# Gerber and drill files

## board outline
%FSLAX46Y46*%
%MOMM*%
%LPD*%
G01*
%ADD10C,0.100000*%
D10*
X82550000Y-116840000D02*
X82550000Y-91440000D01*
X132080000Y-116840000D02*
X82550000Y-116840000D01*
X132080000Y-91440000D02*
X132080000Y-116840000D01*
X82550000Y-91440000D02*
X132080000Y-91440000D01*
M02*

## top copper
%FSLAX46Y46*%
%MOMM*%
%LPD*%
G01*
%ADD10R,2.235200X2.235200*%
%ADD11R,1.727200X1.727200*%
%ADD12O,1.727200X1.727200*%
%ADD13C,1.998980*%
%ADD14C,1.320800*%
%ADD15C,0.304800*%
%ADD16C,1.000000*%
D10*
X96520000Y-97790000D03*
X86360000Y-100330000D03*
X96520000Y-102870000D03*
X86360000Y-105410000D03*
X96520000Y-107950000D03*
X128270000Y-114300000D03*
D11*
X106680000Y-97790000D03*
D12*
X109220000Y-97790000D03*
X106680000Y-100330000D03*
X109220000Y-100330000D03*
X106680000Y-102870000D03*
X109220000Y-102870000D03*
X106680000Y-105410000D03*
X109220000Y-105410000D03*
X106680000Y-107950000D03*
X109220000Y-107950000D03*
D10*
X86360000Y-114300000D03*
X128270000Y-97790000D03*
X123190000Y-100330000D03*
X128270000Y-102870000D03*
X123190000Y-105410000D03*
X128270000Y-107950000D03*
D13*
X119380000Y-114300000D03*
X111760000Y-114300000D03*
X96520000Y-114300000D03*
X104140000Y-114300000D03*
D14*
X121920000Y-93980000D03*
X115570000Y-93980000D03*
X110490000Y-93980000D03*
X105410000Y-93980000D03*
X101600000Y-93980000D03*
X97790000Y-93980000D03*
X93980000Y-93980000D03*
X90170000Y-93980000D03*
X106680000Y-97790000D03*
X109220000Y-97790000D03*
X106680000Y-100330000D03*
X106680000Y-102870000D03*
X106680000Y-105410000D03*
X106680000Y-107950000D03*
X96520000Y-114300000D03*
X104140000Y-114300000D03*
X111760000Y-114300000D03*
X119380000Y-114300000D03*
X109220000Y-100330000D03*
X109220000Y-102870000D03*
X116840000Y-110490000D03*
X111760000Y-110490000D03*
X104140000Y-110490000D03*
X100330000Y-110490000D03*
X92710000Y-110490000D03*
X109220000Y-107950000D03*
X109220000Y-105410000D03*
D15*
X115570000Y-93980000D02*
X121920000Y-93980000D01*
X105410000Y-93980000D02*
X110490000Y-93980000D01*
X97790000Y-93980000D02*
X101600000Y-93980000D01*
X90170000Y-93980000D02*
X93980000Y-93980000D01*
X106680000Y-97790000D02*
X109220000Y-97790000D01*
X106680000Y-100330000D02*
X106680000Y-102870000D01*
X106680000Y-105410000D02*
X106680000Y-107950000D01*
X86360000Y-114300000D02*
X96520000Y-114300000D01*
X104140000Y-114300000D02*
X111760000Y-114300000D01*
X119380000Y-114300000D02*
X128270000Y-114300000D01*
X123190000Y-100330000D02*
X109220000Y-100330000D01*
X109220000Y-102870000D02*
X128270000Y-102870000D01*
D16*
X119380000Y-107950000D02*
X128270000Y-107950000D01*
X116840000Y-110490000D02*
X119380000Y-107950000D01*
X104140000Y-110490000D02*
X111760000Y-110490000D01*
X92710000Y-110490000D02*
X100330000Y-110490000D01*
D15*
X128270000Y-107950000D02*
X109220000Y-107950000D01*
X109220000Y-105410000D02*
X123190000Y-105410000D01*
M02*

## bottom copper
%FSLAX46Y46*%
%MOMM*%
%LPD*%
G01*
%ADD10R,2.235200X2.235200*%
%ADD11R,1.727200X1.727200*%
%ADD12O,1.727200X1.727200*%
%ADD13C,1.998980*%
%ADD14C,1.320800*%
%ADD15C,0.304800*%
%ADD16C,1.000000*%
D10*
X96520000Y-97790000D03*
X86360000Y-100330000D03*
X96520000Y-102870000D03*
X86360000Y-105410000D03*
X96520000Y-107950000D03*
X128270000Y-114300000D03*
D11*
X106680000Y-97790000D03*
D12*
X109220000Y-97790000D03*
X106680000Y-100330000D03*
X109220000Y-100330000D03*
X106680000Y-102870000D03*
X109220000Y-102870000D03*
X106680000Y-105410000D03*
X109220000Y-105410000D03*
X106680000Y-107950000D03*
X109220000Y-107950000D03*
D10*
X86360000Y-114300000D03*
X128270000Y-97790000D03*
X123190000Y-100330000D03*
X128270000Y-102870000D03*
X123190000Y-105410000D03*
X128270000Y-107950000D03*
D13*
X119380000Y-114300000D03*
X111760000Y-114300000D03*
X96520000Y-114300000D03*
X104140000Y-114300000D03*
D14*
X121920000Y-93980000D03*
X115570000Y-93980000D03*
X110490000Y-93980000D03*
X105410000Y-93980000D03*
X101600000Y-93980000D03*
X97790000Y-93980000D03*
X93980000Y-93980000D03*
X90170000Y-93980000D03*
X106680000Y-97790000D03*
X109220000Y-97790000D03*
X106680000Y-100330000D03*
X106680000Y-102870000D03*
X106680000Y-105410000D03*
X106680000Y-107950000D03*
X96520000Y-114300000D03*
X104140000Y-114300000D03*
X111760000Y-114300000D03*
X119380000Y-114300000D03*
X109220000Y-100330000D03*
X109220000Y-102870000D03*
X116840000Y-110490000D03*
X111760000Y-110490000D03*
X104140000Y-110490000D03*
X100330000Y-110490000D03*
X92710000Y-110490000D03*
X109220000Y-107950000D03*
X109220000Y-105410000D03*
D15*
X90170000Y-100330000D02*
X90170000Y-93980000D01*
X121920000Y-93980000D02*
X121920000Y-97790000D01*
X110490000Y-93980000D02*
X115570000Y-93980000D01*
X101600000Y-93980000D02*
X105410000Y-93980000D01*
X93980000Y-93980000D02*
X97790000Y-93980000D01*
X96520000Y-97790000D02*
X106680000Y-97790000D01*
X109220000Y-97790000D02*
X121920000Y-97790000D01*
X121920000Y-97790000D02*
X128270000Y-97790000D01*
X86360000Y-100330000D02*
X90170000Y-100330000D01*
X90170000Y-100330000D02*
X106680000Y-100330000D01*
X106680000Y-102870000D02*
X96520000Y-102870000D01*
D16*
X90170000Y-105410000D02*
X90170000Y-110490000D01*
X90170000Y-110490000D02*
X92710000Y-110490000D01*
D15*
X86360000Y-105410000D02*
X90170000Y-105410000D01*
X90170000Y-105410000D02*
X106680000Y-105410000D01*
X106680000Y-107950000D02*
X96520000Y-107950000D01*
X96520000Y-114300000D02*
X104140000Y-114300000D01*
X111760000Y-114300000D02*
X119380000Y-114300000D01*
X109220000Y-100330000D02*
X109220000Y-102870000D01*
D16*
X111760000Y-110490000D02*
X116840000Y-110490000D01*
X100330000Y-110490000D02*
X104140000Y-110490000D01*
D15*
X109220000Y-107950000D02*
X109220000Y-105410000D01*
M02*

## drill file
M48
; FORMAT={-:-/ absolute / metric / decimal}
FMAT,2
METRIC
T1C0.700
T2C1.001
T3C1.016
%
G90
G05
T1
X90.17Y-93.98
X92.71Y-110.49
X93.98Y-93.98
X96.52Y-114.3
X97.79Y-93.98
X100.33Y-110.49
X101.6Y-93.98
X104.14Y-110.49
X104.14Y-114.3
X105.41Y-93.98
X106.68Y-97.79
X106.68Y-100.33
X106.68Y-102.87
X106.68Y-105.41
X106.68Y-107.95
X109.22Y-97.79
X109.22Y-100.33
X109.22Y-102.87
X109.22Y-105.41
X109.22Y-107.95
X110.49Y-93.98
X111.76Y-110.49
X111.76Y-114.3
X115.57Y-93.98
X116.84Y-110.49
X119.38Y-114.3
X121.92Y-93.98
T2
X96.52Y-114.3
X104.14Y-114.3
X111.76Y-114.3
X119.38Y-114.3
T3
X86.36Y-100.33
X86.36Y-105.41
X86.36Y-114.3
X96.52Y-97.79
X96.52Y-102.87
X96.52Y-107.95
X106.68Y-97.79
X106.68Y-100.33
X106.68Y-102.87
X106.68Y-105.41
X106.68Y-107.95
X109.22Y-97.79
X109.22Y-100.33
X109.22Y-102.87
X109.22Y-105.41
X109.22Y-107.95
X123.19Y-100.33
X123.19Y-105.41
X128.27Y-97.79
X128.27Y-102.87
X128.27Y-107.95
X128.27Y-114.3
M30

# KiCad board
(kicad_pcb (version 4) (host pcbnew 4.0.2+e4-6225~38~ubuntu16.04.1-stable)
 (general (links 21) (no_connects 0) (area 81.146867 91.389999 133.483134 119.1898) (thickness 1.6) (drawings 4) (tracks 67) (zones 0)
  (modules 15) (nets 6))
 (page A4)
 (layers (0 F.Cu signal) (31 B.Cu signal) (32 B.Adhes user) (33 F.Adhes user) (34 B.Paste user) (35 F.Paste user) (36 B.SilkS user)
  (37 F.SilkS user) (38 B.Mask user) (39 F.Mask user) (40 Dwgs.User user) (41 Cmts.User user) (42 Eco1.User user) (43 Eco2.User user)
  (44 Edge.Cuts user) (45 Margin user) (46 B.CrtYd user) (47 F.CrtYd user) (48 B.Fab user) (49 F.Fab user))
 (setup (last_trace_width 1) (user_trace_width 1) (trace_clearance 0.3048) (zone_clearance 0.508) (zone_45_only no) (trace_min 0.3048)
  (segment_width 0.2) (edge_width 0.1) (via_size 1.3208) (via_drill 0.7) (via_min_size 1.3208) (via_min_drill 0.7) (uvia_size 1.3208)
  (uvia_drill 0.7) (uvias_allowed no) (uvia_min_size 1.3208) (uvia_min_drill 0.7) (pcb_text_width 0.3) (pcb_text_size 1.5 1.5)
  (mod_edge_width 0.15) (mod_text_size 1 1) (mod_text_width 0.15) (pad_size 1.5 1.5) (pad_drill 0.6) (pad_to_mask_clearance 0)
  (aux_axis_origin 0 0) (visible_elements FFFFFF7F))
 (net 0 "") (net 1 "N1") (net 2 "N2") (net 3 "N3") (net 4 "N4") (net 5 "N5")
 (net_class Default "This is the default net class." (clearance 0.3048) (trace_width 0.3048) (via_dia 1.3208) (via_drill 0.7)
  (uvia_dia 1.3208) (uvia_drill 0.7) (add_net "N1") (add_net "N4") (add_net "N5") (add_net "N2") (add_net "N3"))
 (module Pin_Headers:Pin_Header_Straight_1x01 (layer F.Cu) (at 96.52 97.79)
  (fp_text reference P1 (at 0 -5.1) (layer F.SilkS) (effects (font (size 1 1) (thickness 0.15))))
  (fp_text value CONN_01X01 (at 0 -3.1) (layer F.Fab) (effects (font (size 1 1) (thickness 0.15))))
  (pad 1 thru_hole rect (at 0 0) (size 2.2352 2.2352) (drill 1.016) (layers *.Cu *.Mask F.SilkS) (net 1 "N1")))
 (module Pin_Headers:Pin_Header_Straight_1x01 (layer F.Cu) (at 86.36 100.33)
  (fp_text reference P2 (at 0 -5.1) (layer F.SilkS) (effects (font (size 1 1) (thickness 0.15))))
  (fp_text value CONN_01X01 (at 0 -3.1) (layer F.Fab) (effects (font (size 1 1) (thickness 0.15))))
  (pad 1 thru_hole rect (at 0 0) (size 2.2352 2.2352) (drill 1.016) (layers *.Cu *.Mask F.SilkS) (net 1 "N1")))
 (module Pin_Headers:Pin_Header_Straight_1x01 (layer F.Cu) (at 96.52 102.87)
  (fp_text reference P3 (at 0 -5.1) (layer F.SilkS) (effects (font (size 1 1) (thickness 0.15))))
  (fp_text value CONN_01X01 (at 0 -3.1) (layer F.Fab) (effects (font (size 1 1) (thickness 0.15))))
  (pad 1 thru_hole rect (at 0 0) (size 2.2352 2.2352) (drill 1.016) (layers *.Cu *.Mask F.SilkS) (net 1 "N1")))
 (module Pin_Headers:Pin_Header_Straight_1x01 (layer F.Cu) (at 86.36 105.41)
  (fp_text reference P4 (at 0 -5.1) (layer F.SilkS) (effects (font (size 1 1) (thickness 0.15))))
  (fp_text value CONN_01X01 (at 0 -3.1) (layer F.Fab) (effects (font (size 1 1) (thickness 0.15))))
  (pad 1 thru_hole rect (at 0 0) (size 2.2352 2.2352) (drill 1.016) (layers *.Cu *.Mask F.SilkS) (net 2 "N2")))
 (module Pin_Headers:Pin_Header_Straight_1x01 (layer F.Cu) (at 96.52 107.95)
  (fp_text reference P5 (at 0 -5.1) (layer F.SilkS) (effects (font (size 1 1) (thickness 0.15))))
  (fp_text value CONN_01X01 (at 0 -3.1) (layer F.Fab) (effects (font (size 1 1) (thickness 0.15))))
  (pad 1 thru_hole rect (at 0 0) (size 2.2352 2.2352) (drill 1.016) (layers *.Cu *.Mask F.SilkS) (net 2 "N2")))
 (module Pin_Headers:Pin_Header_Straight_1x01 (layer F.Cu) (at 128.27 114.3)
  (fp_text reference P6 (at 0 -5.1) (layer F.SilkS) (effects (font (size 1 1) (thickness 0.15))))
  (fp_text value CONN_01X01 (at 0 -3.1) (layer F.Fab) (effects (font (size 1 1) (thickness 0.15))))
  (pad 1 thru_hole rect (at 0 0) (size 2.2352 2.2352) (drill 1.016) (layers *.Cu *.Mask F.SilkS) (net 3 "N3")))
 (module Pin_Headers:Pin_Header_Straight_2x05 (layer F.Cu) (at 106.68 97.79)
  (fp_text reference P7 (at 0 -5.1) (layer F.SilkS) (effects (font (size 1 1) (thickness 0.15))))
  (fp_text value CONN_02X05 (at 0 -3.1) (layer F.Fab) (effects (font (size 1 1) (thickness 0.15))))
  (pad 1 thru_hole rect (at 0 0) (size 1.7272 1.7272) (drill 1.016) (layers *.Cu *.Mask F.SilkS) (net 1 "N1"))
  (pad 2 thru_hole oval (at 2.54 0) (size 1.7272 1.7272) (drill 1.016) (layers *.Cu *.Mask F.SilkS) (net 1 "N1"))
  (pad 3 thru_hole oval (at 0 2.54) (size 1.7272 1.7272) (drill 1.016) (layers *.Cu *.Mask F.SilkS) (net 1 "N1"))
  (pad 4 thru_hole oval (at 2.54 2.54) (size 1.7272 1.7272) (drill 1.016) (layers *.Cu *.Mask F.SilkS) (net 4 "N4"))
  (pad 5 thru_hole oval (at 0 5.08) (size 1.7272 1.7272) (drill 1.016) (layers *.Cu *.Mask F.SilkS) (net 1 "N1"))
  (pad 6 thru_hole oval (at 2.54 5.08) (size 1.7272 1.7272) (drill 1.016) (layers *.Cu *.Mask F.SilkS) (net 4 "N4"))
  (pad 7 thru_hole oval (at 0 7.62) (size 1.7272 1.7272) (drill 1.016) (layers *.Cu *.Mask F.SilkS) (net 2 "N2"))
  (pad 8 thru_hole oval (at 2.54 7.62) (size 1.7272 1.7272) (drill 1.016) (layers *.Cu *.Mask F.SilkS) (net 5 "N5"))
  (pad 9 thru_hole oval (at 0 10.16) (size 1.7272 1.7272) (drill 1.016) (layers *.Cu *.Mask F.SilkS) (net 2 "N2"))
  (pad 10 thru_hole oval (at 2.54 10.16) (size 1.7272 1.7272) (drill 1.016) (layers *.Cu *.Mask F.SilkS) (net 5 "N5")))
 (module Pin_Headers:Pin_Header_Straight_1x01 (layer F.Cu) (at 86.36 114.3)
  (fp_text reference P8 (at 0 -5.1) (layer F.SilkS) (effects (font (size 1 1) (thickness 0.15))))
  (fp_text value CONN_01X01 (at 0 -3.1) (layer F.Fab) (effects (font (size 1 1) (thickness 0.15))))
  (pad 1 thru_hole rect (at 0 0) (size 2.2352 2.2352) (drill 1.016) (layers *.Cu *.Mask F.SilkS) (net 3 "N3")))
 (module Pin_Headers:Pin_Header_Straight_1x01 (layer F.Cu) (at 128.27 97.79)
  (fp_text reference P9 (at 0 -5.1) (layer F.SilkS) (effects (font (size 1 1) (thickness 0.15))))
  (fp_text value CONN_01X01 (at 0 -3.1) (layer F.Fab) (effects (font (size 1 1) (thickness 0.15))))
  (pad 1 thru_hole rect (at 0 0) (size 2.2352 2.2352) (drill 1.016) (layers *.Cu *.Mask F.SilkS) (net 1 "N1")))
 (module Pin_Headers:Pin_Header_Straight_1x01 (layer F.Cu) (at 123.19 100.33)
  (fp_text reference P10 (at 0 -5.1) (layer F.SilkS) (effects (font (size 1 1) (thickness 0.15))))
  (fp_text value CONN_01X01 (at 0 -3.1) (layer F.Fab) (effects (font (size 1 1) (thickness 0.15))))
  (pad 1 thru_hole rect (at 0 0) (size 2.2352 2.2352) (drill 1.016) (layers *.Cu *.Mask F.SilkS) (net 4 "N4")))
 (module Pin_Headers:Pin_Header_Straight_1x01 (layer F.Cu) (at 128.27 102.87)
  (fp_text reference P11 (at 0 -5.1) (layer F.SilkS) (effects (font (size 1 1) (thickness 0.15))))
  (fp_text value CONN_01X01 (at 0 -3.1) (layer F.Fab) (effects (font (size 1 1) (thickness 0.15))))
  (pad 1 thru_hole rect (at 0 0) (size 2.2352 2.2352) (drill 1.016) (layers *.Cu *.Mask F.SilkS) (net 4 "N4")))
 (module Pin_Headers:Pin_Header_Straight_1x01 (layer F.Cu) (at 123.19 105.41)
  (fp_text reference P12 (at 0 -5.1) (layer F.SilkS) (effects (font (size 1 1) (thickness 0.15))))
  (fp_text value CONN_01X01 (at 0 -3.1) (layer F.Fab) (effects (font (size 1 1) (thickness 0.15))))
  (pad 1 thru_hole rect (at 0 0) (size 2.2352 2.2352) (drill 1.016) (layers *.Cu *.Mask F.SilkS) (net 5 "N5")))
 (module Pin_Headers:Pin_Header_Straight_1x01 (layer F.Cu) (at 128.27 107.95)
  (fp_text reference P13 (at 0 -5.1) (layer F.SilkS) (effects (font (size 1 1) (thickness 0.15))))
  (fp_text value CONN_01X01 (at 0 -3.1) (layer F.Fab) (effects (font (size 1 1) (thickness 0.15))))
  (pad 1 thru_hole rect (at 0 0) (size 2.2352 2.2352) (drill 1.016) (layers *.Cu *.Mask F.SilkS) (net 5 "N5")))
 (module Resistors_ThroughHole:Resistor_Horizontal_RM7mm (layer F.Cu) (at 119.38 114.3 180)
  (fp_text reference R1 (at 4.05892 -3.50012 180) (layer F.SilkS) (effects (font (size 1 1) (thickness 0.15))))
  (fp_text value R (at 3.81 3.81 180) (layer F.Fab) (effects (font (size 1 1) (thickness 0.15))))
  (pad 1 thru_hole circle (at 0 0 180) (size 1.99898 1.99898) (drill 1.00076) (layers *.Cu *.SilkS *.Mask) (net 3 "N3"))
  (pad 2 thru_hole circle (at 7.62 0 180) (size 1.99898 1.99898) (drill 1.00076) (layers *.Cu *.SilkS *.Mask) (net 3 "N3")))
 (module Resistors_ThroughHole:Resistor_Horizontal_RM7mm (layer F.Cu) (at 96.52 114.3)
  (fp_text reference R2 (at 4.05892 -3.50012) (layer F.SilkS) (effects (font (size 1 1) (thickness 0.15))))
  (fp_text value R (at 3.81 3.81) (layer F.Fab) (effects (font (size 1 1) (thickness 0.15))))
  (pad 1 thru_hole circle (at 0 0) (size 1.99898 1.99898) (drill 1.00076) (layers *.Cu *.SilkS *.Mask) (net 3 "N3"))
  (pad 2 thru_hole circle (at 7.62 0) (size 1.99898 1.99898) (drill 1.00076) (layers *.Cu *.SilkS *.Mask) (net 3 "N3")))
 (gr_line (start 82.55 116.84) (end 82.55 91.44) (angle 90) (layer Edge.Cuts) (width 0.1))
 (gr_line (start 132.08 116.84) (end 82.55 116.84) (angle 90) (layer Edge.Cuts) (width 0.1))
 (gr_line (start 132.08 91.44) (end 132.08 116.84) (angle 90) (layer Edge.Cuts) (width 0.1))
 (gr_line (start 82.55 91.44) (end 132.08 91.44) (angle 90) (layer Edge.Cuts) (width 0.1))
 (segment (start 90.17 100.33) (end 90.17 93.98) (width 0.3048) (layer B.Cu) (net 1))
 (segment (start 121.92 93.98) (end 121.92 97.79) (width 0.3048) (layer B.Cu) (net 1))
 (via (at 121.92 93.98) (size 1.3208) (drill 0.7) (layers F.Cu B.Cu) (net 1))
 (segment (start 115.57 93.98) (end 121.92 93.98) (width 0.3048) (layer F.Cu) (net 1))
 (via (at 115.57 93.98) (size 1.3208) (drill 0.7) (layers F.Cu B.Cu) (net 1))
 (segment (start 110.49 93.98) (end 115.57 93.98) (width 0.3048) (layer B.Cu) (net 1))
 (via (at 110.49 93.98) (size 1.3208) (drill 0.7) (layers F.Cu B.Cu) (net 1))
 (segment (start 105.41 93.98) (end 110.49 93.98) (width 0.3048) (layer F.Cu) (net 1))
 (via (at 105.41 93.98) (size 1.3208) (drill 0.7) (layers F.Cu B.Cu) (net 1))
 (segment (start 101.6 93.98) (end 105.41 93.98) (width 0.3048) (layer B.Cu) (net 1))
 (via (at 101.6 93.98) (size 1.3208) (drill 0.7) (layers F.Cu B.Cu) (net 1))
 (segment (start 97.79 93.98) (end 101.6 93.98) (width 0.3048) (layer F.Cu) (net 1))
 (via (at 97.79 93.98) (size 1.3208) (drill 0.7) (layers F.Cu B.Cu) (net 1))
 (segment (start 93.98 93.98) (end 97.79 93.98) (width 0.3048) (layer B.Cu) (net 1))
 (via (at 93.98 93.98) (size 1.3208) (drill 0.7) (layers F.Cu B.Cu) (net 1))
 (segment (start 90.17 93.98) (end 93.98 93.98) (width 0.3048) (layer F.Cu) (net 1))
 (via (at 90.17 93.98) (size 1.3208) (drill 0.7) (layers F.Cu B.Cu) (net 1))
 (segment (start 96.52 97.79) (end 106.68 97.79) (width 0.3048) (layer B.Cu) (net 1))
 (via (at 106.68 97.79) (size 1.3208) (drill 0.7) (layers F.Cu B.Cu) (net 1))
 (segment (start 106.68 97.79) (end 109.22 97.79) (width 0.3048) (layer F.Cu) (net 1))
 (via (at 109.22 97.79) (size 1.3208) (drill 0.7) (layers F.Cu B.Cu) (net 1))
 (segment (start 109.22 97.79) (end 121.92 97.79) (width 0.3048) (layer B.Cu) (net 1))
 (segment (start 121.92 97.79) (end 128.27 97.79) (width 0.3048) (layer B.Cu) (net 1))
 (segment (start 86.36 100.33) (end 90.17 100.33) (width 0.3048) (layer B.Cu) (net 1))
 (segment (start 90.17 100.33) (end 106.68 100.33) (width 0.3048) (layer B.Cu) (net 1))
 (via (at 106.68 100.33) (size 1.3208) (drill 0.7) (layers F.Cu B.Cu) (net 1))
 (segment (start 106.68 100.33) (end 106.68 102.87) (width 0.3048) (layer F.Cu) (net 1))
 (via (at 106.68 102.87) (size 1.3208) (drill 0.7) (layers F.Cu B.Cu) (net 1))
 (segment (start 106.68 102.87) (end 96.52 102.87) (width 0.3048) (layer B.Cu) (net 1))
 (segment (start 90.17 105.41) (end 90.17 110.49) (width 1) (layer B.Cu) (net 2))
 (segment (start 90.17 110.49) (end 92.71 110.49) (width 1) (layer B.Cu) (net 2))
 (segment (start 86.36 105.41) (end 90.17 105.41) (width 0.3048) (layer B.Cu) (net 2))
 (segment (start 90.17 105.41) (end 106.68 105.41) (width 0.3048) (layer B.Cu) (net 2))
 (via (at 106.68 105.41) (size 1.3208) (drill 0.7) (layers F.Cu B.Cu) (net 2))
 (segment (start 106.68 105.41) (end 106.68 107.95) (width 0.3048) (layer F.Cu) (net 2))
 (via (at 106.68 107.95) (size 1.3208) (drill 0.7) (layers F.Cu B.Cu) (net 2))
 (segment (start 106.68 107.95) (end 96.52 107.95) (width 0.3048) (layer B.Cu) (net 2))
 (segment (start 86.36 114.3) (end 96.52 114.3) (width 0.3048) (layer F.Cu) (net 3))
 (via (at 96.52 114.3) (size 1.3208) (drill 0.7) (layers F.Cu B.Cu) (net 3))
 (segment (start 96.52 114.3) (end 104.14 114.3) (width 0.3048) (layer B.Cu) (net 3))
 (via (at 104.14 114.3) (size 1.3208) (drill 0.7) (layers F.Cu B.Cu) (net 3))
 (segment (start 104.14 114.3) (end 111.76 114.3) (width 0.3048) (layer F.Cu) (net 3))
 (via (at 111.76 114.3) (size 1.3208) (drill 0.7) (layers F.Cu B.Cu) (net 3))
 (segment (start 111.76 114.3) (end 119.38 114.3) (width 0.3048) (layer B.Cu) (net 3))
 (via (at 119.38 114.3) (size 1.3208) (drill 0.7) (layers F.Cu B.Cu) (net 3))
 (segment (start 119.38 114.3) (end 128.27 114.3) (width 0.3048) (layer F.Cu) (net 3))
 (segment (start 123.19 100.33) (end 109.22 100.33) (width 0.3048) (layer F.Cu) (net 4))
 (via (at 109.22 100.33) (size 1.3208) (drill 0.7) (layers F.Cu B.Cu) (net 4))
 (segment (start 109.22 100.33) (end 109.22 102.87) (width 0.3048) (layer B.Cu) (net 4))
 (via (at 109.22 102.87) (size 1.3208) (drill 0.7) (layers F.Cu B.Cu) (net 4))
 (segment (start 109.22 102.87) (end 128.27 102.87) (width 0.3048) (layer F.Cu) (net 4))
 (segment (start 119.38 107.95) (end 128.27 107.95) (width 1) (layer F.Cu) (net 5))
 (segment (start 116.84 110.49) (end 119.38 107.95) (width 1) (layer F.Cu) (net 5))
 (via (at 116.84 110.49) (size 1.3208) (drill 0.7) (layers F.Cu B.Cu) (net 5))
 (segment (start 111.76 110.49) (end 116.84 110.49) (width 1) (layer B.Cu) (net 5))
 (via (at 111.76 110.49) (size 1.3208) (drill 0.7) (layers F.Cu B.Cu) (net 5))
 (segment (start 104.14 110.49) (end 111.76 110.49) (width 1) (layer F.Cu) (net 5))
 (via (at 104.14 110.49) (size 1.3208) (drill 0.7) (layers F.Cu B.Cu) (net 5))
 (segment (start 100.33 110.49) (end 104.14 110.49) (width 1) (layer B.Cu) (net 5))
 (via (at 100.33 110.49) (size 1.3208) (drill 0.7) (layers F.Cu B.Cu) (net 5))
 (segment (start 92.71 110.49) (end 100.33 110.49) (width 1) (layer F.Cu) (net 5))
 (via (at 92.71 110.49) (size 1.3208) (drill 0.7) (layers F.Cu B.Cu) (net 5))
 (segment (start 128.27 107.95) (end 109.22 107.95) (width 0.3048) (layer F.Cu) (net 5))
 (via (at 109.22 107.95) (size 1.3208) (drill 0.7) (layers F.Cu B.Cu) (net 5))
 (segment (start 109.22 107.95) (end 109.22 105.41) (width 0.3048) (layer B.Cu) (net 5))
 (via (at 109.22 105.41) (size 1.3208) (drill 0.7) (layers F.Cu B.Cu) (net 5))
 (segment (start 109.22 105.41) (end 123.19 105.41) (width 0.3048) (layer F.Cu) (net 5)))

